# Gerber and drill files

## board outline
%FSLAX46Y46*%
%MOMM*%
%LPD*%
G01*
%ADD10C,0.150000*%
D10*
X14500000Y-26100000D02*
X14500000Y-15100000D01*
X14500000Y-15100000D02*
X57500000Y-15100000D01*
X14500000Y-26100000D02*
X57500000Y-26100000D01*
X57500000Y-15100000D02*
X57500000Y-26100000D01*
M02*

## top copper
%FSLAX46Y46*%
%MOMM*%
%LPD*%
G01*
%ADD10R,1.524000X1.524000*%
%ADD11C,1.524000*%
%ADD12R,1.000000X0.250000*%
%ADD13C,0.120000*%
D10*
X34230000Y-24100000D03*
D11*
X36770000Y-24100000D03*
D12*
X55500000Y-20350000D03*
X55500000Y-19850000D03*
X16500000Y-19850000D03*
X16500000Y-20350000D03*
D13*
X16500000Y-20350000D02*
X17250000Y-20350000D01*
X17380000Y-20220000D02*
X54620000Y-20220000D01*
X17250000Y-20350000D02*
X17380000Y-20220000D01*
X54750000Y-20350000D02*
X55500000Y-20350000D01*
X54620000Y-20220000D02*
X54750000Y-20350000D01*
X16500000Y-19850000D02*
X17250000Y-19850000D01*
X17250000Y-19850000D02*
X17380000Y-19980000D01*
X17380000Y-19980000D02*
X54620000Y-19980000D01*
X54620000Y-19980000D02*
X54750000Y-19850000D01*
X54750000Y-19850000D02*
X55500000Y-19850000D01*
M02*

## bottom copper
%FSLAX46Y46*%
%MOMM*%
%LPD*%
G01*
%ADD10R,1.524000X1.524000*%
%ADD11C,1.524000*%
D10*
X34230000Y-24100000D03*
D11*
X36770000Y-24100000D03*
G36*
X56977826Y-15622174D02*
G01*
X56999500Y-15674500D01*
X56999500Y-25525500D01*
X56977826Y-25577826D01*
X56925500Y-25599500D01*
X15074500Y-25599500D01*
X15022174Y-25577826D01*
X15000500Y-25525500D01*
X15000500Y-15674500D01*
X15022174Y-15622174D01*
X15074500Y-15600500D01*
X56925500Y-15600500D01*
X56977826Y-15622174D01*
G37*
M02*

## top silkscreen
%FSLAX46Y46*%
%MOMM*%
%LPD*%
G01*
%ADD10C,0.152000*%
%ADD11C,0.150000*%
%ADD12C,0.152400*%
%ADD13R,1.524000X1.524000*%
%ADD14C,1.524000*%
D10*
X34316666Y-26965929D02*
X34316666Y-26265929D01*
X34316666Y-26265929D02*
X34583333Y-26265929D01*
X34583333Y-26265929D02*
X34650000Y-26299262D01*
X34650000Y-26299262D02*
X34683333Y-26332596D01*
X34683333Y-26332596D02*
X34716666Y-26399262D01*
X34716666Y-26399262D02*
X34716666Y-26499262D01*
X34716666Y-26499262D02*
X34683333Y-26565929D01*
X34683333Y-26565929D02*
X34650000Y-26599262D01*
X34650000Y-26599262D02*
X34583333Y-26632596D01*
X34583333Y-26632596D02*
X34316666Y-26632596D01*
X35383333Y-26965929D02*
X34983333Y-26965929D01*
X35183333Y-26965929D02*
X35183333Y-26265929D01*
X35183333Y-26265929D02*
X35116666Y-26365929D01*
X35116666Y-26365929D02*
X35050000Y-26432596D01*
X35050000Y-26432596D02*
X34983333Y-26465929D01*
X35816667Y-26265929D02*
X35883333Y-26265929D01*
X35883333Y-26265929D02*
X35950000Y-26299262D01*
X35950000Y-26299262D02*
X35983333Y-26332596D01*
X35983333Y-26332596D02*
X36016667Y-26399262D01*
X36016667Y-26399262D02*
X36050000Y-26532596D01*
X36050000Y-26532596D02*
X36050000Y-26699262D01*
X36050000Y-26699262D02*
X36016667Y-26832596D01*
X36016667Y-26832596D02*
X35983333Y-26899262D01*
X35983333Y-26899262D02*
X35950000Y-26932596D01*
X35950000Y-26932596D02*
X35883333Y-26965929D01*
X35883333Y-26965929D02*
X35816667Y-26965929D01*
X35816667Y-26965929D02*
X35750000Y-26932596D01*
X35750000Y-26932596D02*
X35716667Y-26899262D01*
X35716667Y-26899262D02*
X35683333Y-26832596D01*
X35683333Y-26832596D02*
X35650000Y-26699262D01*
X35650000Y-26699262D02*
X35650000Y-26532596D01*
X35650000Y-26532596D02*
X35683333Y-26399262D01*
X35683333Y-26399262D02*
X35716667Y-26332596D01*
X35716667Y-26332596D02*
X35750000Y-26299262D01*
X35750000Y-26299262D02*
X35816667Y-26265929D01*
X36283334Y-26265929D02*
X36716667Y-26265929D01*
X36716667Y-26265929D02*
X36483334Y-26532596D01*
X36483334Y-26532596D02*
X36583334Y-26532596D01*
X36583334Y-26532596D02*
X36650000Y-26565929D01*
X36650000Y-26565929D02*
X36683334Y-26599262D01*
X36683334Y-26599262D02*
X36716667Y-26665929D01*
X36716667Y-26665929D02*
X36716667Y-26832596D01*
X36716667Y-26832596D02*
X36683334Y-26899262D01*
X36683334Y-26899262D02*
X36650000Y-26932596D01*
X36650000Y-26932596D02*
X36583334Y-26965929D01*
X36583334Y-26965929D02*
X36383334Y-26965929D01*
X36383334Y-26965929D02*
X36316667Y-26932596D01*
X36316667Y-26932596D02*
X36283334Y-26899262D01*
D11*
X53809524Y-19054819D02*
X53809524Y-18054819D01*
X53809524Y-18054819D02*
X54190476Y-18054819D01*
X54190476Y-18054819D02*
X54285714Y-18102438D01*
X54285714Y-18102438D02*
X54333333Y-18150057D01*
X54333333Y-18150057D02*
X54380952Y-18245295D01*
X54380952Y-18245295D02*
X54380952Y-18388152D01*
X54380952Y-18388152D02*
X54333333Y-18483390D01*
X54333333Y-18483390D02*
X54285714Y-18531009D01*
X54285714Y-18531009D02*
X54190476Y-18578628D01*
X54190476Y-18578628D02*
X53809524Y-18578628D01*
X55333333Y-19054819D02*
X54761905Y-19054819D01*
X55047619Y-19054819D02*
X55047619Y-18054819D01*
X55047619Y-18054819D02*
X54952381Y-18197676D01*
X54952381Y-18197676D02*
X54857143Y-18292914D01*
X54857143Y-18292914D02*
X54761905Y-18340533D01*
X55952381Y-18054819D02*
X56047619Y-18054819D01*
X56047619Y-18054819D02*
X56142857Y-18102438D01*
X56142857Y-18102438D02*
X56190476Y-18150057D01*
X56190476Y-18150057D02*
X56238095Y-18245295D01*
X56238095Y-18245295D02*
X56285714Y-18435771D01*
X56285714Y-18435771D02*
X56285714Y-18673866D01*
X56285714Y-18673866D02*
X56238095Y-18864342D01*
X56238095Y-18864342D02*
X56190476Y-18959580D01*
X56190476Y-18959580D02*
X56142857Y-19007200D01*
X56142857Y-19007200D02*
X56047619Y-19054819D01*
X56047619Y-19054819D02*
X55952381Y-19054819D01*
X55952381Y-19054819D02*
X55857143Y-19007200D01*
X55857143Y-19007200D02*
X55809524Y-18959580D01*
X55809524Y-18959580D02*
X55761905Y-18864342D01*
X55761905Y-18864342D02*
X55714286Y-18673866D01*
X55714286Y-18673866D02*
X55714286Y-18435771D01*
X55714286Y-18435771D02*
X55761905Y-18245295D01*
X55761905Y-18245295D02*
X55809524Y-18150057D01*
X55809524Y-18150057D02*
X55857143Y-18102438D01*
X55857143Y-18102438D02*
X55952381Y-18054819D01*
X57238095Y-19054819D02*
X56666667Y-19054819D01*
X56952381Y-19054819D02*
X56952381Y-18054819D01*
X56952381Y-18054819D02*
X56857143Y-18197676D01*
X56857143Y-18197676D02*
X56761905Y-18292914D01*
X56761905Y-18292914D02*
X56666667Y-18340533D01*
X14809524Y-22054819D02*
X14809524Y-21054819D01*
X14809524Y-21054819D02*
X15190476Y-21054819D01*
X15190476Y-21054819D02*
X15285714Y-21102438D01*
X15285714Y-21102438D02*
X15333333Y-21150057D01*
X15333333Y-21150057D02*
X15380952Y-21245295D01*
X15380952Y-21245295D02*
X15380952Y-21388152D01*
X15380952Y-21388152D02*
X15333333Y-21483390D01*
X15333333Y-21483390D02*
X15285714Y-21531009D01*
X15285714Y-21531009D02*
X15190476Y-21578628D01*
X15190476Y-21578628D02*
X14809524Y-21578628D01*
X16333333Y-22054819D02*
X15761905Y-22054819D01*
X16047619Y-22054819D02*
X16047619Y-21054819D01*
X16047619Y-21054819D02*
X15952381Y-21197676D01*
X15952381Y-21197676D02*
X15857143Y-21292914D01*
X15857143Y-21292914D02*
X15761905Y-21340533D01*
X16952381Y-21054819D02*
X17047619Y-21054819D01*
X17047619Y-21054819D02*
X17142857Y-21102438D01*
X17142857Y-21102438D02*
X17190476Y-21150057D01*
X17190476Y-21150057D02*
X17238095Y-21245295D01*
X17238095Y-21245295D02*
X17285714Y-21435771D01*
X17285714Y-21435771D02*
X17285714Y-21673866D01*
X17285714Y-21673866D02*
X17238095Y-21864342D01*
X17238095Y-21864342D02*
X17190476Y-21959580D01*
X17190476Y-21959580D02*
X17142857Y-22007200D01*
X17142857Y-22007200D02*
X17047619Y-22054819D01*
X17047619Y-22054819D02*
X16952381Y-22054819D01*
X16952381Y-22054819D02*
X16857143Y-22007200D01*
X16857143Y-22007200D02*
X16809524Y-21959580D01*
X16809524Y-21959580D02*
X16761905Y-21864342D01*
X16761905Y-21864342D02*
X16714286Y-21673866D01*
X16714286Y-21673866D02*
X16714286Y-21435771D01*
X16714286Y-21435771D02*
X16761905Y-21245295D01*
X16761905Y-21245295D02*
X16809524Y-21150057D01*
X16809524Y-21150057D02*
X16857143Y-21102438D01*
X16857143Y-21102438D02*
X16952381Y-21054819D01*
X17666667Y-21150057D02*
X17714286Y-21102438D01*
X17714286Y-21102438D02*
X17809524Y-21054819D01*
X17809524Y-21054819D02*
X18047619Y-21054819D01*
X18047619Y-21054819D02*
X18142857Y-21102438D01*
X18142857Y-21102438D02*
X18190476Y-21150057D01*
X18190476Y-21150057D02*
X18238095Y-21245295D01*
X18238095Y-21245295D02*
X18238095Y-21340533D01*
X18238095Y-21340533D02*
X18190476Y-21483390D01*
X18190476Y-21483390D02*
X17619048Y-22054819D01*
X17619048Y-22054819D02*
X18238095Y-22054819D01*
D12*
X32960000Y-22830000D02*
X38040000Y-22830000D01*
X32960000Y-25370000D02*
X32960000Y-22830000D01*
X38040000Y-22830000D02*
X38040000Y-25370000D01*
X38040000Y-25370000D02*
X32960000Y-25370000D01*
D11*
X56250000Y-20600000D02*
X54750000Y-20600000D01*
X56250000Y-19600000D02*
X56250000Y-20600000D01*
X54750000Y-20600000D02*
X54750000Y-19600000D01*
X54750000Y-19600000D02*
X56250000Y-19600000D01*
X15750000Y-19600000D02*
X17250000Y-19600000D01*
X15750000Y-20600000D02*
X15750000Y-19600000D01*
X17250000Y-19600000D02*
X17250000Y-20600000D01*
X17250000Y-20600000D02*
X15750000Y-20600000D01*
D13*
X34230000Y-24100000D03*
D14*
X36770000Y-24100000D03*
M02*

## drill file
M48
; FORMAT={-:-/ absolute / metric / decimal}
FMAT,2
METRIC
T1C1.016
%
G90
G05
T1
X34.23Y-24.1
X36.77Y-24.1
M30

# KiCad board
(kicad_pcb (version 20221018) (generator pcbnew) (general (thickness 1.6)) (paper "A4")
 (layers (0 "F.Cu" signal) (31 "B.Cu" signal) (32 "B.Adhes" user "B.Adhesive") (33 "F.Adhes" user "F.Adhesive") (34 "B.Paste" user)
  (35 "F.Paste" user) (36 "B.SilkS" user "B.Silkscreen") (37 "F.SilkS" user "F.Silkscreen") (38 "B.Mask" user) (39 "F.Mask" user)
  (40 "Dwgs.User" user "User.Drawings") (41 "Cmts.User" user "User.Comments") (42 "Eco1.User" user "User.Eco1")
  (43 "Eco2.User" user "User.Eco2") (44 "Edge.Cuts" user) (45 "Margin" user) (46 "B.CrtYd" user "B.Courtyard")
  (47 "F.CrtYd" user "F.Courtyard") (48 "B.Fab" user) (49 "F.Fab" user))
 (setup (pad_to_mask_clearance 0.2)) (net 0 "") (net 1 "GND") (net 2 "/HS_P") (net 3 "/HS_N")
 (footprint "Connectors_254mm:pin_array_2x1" (layer "F.Cu") (at 35.5 24.1)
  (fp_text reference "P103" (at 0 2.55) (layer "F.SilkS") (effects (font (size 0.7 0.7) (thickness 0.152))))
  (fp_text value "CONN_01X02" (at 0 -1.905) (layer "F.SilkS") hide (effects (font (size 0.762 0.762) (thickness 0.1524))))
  (fp_line (start -2.54 -1.27) (end 2.54 -1.27) (stroke (width 0.1524) (type solid)) (layer "F.SilkS"))
  (fp_line (start -2.54 1.27) (end -2.54 -1.27) (stroke (width 0.1524) (type solid)) (layer "F.SilkS"))
  (fp_line (start 2.54 -1.27) (end 2.54 1.27) (stroke (width 0.1524) (type solid)) (layer "F.SilkS"))
  (fp_line (start 2.54 1.27) (end -2.54 1.27) (stroke (width 0.1524) (type solid)) (layer "F.SilkS"))
  (pad "1" thru_hole rect (at -1.27 0) (size 1.524 1.524) (drill 1.016) (layers "*.Cu" "*.Mask" "F.SilkS") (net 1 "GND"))
  (pad "2" thru_hole circle (at 1.27 0) (size 1.524 1.524) (drill 1.016) (layers "*.Cu" "*.Mask" "F.SilkS") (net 1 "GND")))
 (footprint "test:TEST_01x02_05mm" (layer "F.Cu") (at 55.5 20.1 180)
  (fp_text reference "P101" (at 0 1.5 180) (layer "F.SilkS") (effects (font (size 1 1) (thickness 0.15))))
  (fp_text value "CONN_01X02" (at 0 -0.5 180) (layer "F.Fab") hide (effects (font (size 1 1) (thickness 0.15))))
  (fp_line (start -0.75 -0.5) (end 0.75 -0.5) (stroke (width 0.15) (type solid)) (layer "F.SilkS"))
  (fp_line (start -0.75 0.5) (end -0.75 -0.5) (stroke (width 0.15) (type solid)) (layer "F.SilkS"))
  (fp_line (start 0.75 -0.5) (end 0.75 0.5) (stroke (width 0.15) (type solid)) (layer "F.SilkS"))
  (fp_line (start 0.75 0.5) (end -0.75 0.5) (stroke (width 0.15) (type solid)) (layer "F.SilkS"))
  (pad "1" smd rect (at 0 -0.25 180) (size 1 0.25) (layers "F.Cu" "F.Paste" "F.Mask") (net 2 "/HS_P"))
  (pad "2" smd rect (at 0 0.25 180) (size 1 0.25) (layers "F.Cu" "F.Paste" "F.Mask") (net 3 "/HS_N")))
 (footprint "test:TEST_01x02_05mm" (layer "F.Cu") (at 16.5 20.1)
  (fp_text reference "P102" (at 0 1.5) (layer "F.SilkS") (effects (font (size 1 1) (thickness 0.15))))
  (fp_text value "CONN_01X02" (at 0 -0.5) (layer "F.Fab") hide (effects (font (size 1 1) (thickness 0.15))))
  (fp_line (start -0.75 -0.5) (end 0.75 -0.5) (stroke (width 0.15) (type solid)) (layer "F.SilkS"))
  (fp_line (start -0.75 0.5) (end -0.75 -0.5) (stroke (width 0.15) (type solid)) (layer "F.SilkS"))
  (fp_line (start 0.75 -0.5) (end 0.75 0.5) (stroke (width 0.15) (type solid)) (layer "F.SilkS"))
  (fp_line (start 0.75 0.5) (end -0.75 0.5) (stroke (width 0.15) (type solid)) (layer "F.SilkS"))
  (pad "1" smd rect (at 0 -0.25) (size 1 0.25) (layers "F.Cu" "F.Paste" "F.Mask") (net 3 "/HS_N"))
  (pad "2" smd rect (at 0 0.25) (size 1 0.25) (layers "F.Cu" "F.Paste" "F.Mask") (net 2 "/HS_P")))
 (gr_line (start 14.5 26.1) (end 14.5 15.1) (stroke (width 0.15) (type solid)) (layer "Edge.Cuts"))
 (gr_line (start 14.5 15.1) (end 57.5 15.1) (stroke (width 0.15) (type solid)) (layer "Edge.Cuts"))
 (gr_line (start 14.5 26.1) (end 57.5 26.1) (stroke (width 0.15) (type solid)) (layer "Edge.Cuts"))
 (gr_line (start 57.5 15.1) (end 57.5 26.1) (stroke (width 0.15) (type solid)) (layer "Edge.Cuts"))
 (segment (start 16.5 20.35) (end 17.25 20.35) (width 0.12) (layer "F.Cu") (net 2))
 (segment (start 17.38 20.22) (end 54.62 20.22) (width 0.12) (layer "F.Cu") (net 2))
 (segment (start 17.25 20.35) (end 17.38 20.22) (width 0.12) (layer "F.Cu") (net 2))
 (segment (start 54.75 20.35) (end 55.5 20.35) (width 0.12) (layer "F.Cu") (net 2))
 (segment (start 54.62 20.22) (end 54.75 20.35) (width 0.12) (layer "F.Cu") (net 2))
 (segment (start 16.5 19.85) (end 17.25 19.85) (width 0.12) (layer "F.Cu") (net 3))
 (segment (start 17.25 19.85) (end 17.38 19.98) (width 0.12) (layer "F.Cu") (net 3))
 (segment (start 17.38 19.98) (end 54.62 19.98) (width 0.12) (layer "F.Cu") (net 3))
 (segment (start 54.62 19.98) (end 54.75 19.85) (width 0.12) (layer "F.Cu") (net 3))
 (segment (start 54.75 19.85) (end 55.5 19.85) (width 0.12) (layer "F.Cu") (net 3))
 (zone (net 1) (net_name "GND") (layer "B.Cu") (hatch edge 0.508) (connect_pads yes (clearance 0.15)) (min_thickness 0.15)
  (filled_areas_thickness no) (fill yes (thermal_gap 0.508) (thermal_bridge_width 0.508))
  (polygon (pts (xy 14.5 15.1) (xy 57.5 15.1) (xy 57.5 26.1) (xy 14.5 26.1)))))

